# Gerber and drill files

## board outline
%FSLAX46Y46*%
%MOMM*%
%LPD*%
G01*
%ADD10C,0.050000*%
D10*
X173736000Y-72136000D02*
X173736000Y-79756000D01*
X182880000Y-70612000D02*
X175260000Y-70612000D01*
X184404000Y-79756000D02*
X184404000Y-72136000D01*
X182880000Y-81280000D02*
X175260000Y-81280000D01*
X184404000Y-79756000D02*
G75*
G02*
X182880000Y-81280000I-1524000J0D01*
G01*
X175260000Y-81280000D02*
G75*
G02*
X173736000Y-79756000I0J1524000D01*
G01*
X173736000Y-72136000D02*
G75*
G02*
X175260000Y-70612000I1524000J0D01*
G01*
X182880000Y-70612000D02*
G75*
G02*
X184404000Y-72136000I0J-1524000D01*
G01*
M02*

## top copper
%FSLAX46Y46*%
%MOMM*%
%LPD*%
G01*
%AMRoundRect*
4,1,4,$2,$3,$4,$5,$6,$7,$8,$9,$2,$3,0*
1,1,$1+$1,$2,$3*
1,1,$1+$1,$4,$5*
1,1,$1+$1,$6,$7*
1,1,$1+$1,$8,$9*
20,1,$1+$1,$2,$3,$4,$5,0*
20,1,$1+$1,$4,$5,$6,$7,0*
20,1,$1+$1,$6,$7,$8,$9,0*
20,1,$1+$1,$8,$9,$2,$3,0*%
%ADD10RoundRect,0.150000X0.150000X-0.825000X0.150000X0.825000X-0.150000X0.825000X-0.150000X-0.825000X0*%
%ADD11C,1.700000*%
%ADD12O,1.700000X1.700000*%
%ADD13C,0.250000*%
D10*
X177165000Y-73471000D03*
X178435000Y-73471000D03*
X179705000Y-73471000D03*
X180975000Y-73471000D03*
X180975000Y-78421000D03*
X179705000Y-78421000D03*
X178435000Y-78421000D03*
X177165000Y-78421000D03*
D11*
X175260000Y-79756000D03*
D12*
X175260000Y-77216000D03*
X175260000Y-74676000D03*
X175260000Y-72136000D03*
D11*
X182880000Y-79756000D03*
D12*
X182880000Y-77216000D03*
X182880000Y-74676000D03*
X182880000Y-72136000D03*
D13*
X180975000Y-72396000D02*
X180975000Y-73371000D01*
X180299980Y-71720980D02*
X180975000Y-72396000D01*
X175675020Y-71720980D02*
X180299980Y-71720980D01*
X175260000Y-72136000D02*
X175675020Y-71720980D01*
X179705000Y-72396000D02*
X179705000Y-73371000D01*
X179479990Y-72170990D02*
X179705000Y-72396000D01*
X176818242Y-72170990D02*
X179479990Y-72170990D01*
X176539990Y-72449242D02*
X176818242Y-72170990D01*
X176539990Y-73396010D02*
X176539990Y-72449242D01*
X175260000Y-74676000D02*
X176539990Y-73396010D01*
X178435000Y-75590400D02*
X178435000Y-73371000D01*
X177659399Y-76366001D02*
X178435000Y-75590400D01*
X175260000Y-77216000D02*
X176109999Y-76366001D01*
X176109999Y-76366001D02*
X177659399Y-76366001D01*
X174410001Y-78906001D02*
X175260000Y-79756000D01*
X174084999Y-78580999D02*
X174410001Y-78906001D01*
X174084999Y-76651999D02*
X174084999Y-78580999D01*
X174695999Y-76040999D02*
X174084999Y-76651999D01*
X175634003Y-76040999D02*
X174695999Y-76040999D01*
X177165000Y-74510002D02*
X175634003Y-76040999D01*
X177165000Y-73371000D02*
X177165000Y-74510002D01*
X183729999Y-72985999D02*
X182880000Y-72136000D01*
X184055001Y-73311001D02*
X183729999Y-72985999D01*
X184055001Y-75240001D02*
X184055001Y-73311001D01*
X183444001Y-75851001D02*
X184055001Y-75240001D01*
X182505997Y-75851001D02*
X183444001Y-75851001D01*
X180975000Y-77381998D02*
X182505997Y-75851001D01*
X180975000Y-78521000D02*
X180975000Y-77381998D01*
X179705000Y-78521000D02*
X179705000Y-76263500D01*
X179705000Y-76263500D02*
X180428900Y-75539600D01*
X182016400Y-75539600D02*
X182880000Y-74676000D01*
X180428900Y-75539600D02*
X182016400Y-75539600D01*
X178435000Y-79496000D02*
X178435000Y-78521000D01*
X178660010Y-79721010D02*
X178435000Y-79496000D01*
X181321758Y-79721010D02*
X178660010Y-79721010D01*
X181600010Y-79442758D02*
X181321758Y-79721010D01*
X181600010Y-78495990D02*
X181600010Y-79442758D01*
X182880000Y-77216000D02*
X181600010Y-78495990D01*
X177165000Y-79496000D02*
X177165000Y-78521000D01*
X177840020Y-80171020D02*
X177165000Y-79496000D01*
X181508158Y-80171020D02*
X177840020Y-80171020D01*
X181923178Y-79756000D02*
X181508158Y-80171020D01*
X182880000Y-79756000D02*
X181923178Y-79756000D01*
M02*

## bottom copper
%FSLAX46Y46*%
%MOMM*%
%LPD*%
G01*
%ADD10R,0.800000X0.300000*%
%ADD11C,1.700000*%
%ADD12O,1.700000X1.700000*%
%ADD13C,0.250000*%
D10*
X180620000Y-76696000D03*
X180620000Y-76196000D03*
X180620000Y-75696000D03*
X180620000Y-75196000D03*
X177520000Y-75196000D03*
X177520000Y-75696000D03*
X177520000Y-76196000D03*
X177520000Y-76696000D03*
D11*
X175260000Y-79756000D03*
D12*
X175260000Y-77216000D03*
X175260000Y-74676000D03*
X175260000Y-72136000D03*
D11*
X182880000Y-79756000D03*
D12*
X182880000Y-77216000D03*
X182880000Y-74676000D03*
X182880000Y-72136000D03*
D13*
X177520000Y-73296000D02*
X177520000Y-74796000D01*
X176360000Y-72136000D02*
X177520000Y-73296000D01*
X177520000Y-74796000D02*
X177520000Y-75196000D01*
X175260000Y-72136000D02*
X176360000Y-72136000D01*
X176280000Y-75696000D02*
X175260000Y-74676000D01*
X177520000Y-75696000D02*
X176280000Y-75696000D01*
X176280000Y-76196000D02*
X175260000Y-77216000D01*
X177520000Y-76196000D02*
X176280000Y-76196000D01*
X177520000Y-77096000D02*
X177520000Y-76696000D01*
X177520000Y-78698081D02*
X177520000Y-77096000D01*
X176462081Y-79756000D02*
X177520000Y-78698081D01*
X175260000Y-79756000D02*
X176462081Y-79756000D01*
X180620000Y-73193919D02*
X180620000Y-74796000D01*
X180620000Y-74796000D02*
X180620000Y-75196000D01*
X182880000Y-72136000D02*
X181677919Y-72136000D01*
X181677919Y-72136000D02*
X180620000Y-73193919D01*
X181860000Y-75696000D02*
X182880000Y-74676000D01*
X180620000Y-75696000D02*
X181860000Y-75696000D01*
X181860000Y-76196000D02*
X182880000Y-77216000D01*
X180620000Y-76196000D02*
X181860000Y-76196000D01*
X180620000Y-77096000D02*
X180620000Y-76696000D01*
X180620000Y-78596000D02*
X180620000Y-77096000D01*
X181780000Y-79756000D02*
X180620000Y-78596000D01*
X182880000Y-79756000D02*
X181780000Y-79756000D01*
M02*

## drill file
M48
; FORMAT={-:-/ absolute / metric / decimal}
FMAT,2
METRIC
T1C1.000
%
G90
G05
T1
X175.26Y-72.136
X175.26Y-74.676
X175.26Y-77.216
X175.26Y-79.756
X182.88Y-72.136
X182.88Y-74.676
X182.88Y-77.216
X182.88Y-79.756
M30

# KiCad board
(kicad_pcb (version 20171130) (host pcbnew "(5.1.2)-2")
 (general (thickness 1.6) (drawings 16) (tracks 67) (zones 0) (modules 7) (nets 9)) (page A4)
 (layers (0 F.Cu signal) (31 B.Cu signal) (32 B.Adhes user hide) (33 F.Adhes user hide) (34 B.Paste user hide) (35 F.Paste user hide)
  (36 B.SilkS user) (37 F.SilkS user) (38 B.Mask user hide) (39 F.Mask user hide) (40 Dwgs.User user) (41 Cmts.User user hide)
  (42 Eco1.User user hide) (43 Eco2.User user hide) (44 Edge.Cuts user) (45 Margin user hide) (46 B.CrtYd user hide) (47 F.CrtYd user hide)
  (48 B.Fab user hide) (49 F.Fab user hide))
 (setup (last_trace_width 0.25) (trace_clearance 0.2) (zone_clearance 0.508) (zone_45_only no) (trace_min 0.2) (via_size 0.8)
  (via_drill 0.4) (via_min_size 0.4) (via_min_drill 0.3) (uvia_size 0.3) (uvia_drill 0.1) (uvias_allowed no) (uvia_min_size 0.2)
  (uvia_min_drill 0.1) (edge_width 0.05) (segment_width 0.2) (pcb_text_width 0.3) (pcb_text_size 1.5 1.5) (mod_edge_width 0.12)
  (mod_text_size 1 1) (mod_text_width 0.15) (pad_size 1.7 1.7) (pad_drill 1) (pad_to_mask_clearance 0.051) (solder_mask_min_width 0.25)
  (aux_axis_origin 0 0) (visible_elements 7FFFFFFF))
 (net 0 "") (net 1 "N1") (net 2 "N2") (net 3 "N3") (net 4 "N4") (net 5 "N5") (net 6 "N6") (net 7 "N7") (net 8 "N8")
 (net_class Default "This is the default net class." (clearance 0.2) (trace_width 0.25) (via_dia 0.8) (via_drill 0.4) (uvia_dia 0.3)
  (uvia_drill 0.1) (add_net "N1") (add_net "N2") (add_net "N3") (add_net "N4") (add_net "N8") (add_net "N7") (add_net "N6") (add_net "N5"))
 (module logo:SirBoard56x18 (layer B.Cu) (at 179.07 78.867)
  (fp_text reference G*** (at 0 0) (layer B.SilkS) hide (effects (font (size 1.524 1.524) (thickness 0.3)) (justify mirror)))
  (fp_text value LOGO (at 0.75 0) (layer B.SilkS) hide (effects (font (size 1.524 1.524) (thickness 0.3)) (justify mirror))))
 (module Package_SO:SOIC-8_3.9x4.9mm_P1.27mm (layer F.Cu) (at 179.07 75.946 90)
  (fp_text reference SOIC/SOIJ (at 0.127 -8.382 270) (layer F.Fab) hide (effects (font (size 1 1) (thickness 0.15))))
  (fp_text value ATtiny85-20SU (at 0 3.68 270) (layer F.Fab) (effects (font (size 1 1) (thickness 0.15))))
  (pad 8 smd roundrect (at 2.475 -1.905 90) (size 1.95 0.6) (layers F.Cu F.Paste F.Mask) (roundrect_rratio 0.25) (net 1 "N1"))
  (pad 7 smd roundrect (at 2.475 -0.635 90) (size 1.95 0.6) (layers F.Cu F.Paste F.Mask) (roundrect_rratio 0.25) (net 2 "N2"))
  (pad 6 smd roundrect (at 2.475 0.635 90) (size 1.95 0.6) (layers F.Cu F.Paste F.Mask) (roundrect_rratio 0.25) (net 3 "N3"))
  (pad 5 smd roundrect (at 2.475 1.905 90) (size 1.95 0.6) (layers F.Cu F.Paste F.Mask) (roundrect_rratio 0.25) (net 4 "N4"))
  (pad 4 smd roundrect (at -2.475 1.905 90) (size 1.95 0.6) (layers F.Cu F.Paste F.Mask) (roundrect_rratio 0.25) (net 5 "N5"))
  (pad 3 smd roundrect (at -2.475 0.635 90) (size 1.95 0.6) (layers F.Cu F.Paste F.Mask) (roundrect_rratio 0.25) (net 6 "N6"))
  (pad 2 smd roundrect (at -2.475 -0.635 90) (size 1.95 0.6) (layers F.Cu F.Paste F.Mask) (roundrect_rratio 0.25) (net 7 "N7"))
  (pad 1 smd roundrect (at -2.475 -1.905 90) (size 1.95 0.6) (layers F.Cu F.Paste F.Mask) (roundrect_rratio 0.25) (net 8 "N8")))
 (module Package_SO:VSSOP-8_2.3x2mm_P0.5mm (layer B.Cu) (at 179.07 75.946)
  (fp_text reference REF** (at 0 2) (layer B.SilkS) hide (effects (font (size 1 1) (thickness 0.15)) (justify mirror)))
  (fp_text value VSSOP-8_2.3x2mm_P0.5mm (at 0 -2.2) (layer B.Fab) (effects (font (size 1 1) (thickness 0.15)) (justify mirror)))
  (pad 8 smd rect (at 1.55 0.75 90) (size 0.3 0.8) (layers B.Cu B.Paste B.Mask) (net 8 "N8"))
  (pad 7 smd rect (at 1.55 0.25 90) (size 0.3 0.8) (layers B.Cu B.Paste B.Mask) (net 7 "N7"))
  (pad 6 smd rect (at 1.55 -0.25 90) (size 0.3 0.8) (layers B.Cu B.Paste B.Mask) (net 6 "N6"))
  (pad 5 smd rect (at 1.55 -0.75 90) (size 0.3 0.8) (layers B.Cu B.Paste B.Mask) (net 5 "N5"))
  (pad 4 smd rect (at -1.55 -0.75 90) (size 0.3 0.8) (layers B.Cu B.Paste B.Mask) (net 4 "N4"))
  (pad 3 smd rect (at -1.55 -0.25 90) (size 0.3 0.8) (layers B.Cu B.Paste B.Mask) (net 3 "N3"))
  (pad 2 smd rect (at -1.55 0.25 90) (size 0.3 0.8) (layers B.Cu B.Paste B.Mask) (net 2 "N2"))
  (pad 1 smd rect (at -1.55 0.75 90) (size 0.3 0.8) (layers B.Cu B.Paste B.Mask) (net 1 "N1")))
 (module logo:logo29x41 (layer F.Cu) (at 179.07 71.501 90)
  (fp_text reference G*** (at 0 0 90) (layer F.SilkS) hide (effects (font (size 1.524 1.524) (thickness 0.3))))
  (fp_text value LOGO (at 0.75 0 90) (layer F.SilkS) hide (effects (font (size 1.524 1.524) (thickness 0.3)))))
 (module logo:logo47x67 (layer B.Cu) (at 179.07 72.5805 90)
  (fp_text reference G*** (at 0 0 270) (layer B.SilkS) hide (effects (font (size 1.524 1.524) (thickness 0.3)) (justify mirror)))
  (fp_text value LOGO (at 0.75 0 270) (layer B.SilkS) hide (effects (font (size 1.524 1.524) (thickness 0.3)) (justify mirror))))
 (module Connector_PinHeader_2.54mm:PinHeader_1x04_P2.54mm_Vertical (layer B.Cu) (at 175.26 79.756)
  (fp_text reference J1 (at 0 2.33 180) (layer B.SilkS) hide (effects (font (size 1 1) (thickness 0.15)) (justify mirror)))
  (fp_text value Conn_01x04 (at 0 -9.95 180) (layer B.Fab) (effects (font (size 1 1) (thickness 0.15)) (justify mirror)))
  (pad 1 thru_hole circle (at 0 0) (size 1.7 1.7) (drill 1) (layers *.Cu *.Mask) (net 1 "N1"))
  (pad 2 thru_hole oval (at 0 -2.54) (size 1.7 1.7) (drill 1) (layers *.Cu *.Mask) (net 2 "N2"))
  (pad 3 thru_hole oval (at 0 -5.08) (size 1.7 1.7) (drill 1) (layers *.Cu *.Mask) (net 3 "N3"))
  (pad 4 thru_hole oval (at 0 -7.62) (size 1.7 1.7) (drill 1) (layers *.Cu *.Mask) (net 4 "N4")))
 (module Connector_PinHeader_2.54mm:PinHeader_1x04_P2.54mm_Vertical (layer B.Cu) (at 182.88 79.756)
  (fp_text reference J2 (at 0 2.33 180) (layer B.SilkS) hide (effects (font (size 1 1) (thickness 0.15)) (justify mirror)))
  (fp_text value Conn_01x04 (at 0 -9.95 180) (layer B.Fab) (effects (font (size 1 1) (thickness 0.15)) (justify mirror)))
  (pad 1 thru_hole circle (at 0 0) (size 1.7 1.7) (drill 1) (layers *.Cu *.Mask) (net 8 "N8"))
  (pad 2 thru_hole oval (at 0 -2.54) (size 1.7 1.7) (drill 1) (layers *.Cu *.Mask) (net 7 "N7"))
  (pad 3 thru_hole oval (at 0 -5.08) (size 1.7 1.7) (drill 1) (layers *.Cu *.Mask) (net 6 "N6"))
  (pad 4 thru_hole oval (at 0 -7.62) (size 1.7 1.7) (drill 1) (layers *.Cu *.Mask) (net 5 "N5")))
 (gr_line (start 173.736 72.136) (end 173.736 79.756) (layer Edge.Cuts) (width 0.05))
 (gr_line (start 182.88 70.612) (end 175.26 70.612) (layer Edge.Cuts) (width 0.05))
 (gr_line (start 184.404 79.756) (end 184.404 72.136) (layer Edge.Cuts) (width 0.05))
 (gr_line (start 182.88 81.28) (end 175.26 81.28) (layer Edge.Cuts) (width 0.05))
 (gr_arc (start 182.88 79.756) (end 182.88 81.28) (angle -90) (layer Edge.Cuts) (width 0.05))
 (gr_arc (start 175.26 79.756) (end 173.736 79.756) (angle -90) (layer Edge.Cuts) (width 0.05))
 (gr_arc (start 175.26 72.136) (end 175.26 70.612) (angle -90) (layer Edge.Cuts) (width 0.05))
 (gr_arc (start 182.88 72.136) (end 184.404 72.136) (angle -90) (layer Edge.Cuts) (width 0.05))
 (segment (start 180.975 72.396) (end 180.975 73.371) (width 0.25) (layer F.Cu) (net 4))
 (segment (start 180.29998 71.72098) (end 180.975 72.396) (width 0.25) (layer F.Cu) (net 4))
 (segment (start 175.67502 71.72098) (end 180.29998 71.72098) (width 0.25) (layer F.Cu) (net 4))
 (segment (start 175.26 72.136) (end 175.67502 71.72098) (width 0.25) (layer F.Cu) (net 4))
 (segment (start 177.52 73.296) (end 177.52 74.796) (width 0.25) (layer B.Cu) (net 4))
 (segment (start 176.36 72.136) (end 177.52 73.296) (width 0.25) (layer B.Cu) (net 4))
 (segment (start 177.52 74.796) (end 177.52 75.196) (width 0.25) (layer B.Cu) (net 4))
 (segment (start 175.26 72.136) (end 176.36 72.136) (width 0.25) (layer B.Cu) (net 4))
 (segment (start 179.705 72.396) (end 179.705 73.371) (width 0.25) (layer F.Cu) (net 3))
 (segment (start 179.47999 72.17099) (end 179.705 72.396) (width 0.25) (layer F.Cu) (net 3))
 (segment (start 176.818242 72.17099) (end 179.47999 72.17099) (width 0.25) (layer F.Cu) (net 3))
 (segment (start 176.53999 72.449242) (end 176.818242 72.17099) (width 0.25) (layer F.Cu) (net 3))
 (segment (start 176.53999 73.39601) (end 176.53999 72.449242) (width 0.25) (layer F.Cu) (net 3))
 (segment (start 175.26 74.676) (end 176.53999 73.39601) (width 0.25) (layer F.Cu) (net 3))
 (segment (start 176.28 75.696) (end 175.26 74.676) (width 0.25) (layer B.Cu) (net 3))
 (segment (start 177.52 75.696) (end 176.28 75.696) (width 0.25) (layer B.Cu) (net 3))
 (segment (start 178.435 75.5904) (end 178.435 73.371) (width 0.25) (layer F.Cu) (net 2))
 (segment (start 177.659399 76.366001) (end 178.435 75.5904) (width 0.25) (layer F.Cu) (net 2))
 (segment (start 175.26 77.216) (end 176.109999 76.366001) (width 0.25) (layer F.Cu) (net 2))
 (segment (start 176.109999 76.366001) (end 177.659399 76.366001) (width 0.25) (layer F.Cu) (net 2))
 (segment (start 176.28 76.196) (end 175.26 77.216) (width 0.25) (layer B.Cu) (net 2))
 (segment (start 177.52 76.196) (end 176.28 76.196) (width 0.25) (layer B.Cu) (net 2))
 (segment (start 174.410001 78.906001) (end 175.26 79.756) (width 0.25) (layer F.Cu) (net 1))
 (segment (start 174.084999 78.580999) (end 174.410001 78.906001) (width 0.25) (layer F.Cu) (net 1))
 (segment (start 174.084999 76.651999) (end 174.084999 78.580999) (width 0.25) (layer F.Cu) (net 1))
 (segment (start 174.695999 76.040999) (end 174.084999 76.651999) (width 0.25) (layer F.Cu) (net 1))
 (segment (start 175.634003 76.040999) (end 174.695999 76.040999) (width 0.25) (layer F.Cu) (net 1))
 (segment (start 177.165 74.510002) (end 175.634003 76.040999) (width 0.25) (layer F.Cu) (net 1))
 (segment (start 177.165 73.371) (end 177.165 74.510002) (width 0.25) (layer F.Cu) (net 1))
 (segment (start 177.52 77.096) (end 177.52 76.696) (width 0.25) (layer B.Cu) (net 1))
 (segment (start 177.52 78.698081) (end 177.52 77.096) (width 0.25) (layer B.Cu) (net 1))
 (segment (start 176.462081 79.756) (end 177.52 78.698081) (width 0.25) (layer B.Cu) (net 1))
 (segment (start 175.26 79.756) (end 176.462081 79.756) (width 0.25) (layer B.Cu) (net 1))
 (segment (start 180.62 73.193919) (end 180.62 74.796) (width 0.25) (layer B.Cu) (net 5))
 (segment (start 180.62 74.796) (end 180.62 75.196) (width 0.25) (layer B.Cu) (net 5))
 (segment (start 182.88 72.136) (end 181.677919 72.136) (width 0.25) (layer B.Cu) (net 5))
 (segment (start 181.677919 72.136) (end 180.62 73.193919) (width 0.25) (layer B.Cu) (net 5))
 (segment (start 183.729999 72.985999) (end 182.88 72.136) (width 0.25) (layer F.Cu) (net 5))
 (segment (start 184.055001 73.311001) (end 183.729999 72.985999) (width 0.25) (layer F.Cu) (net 5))
 (segment (start 184.055001 75.240001) (end 184.055001 73.311001) (width 0.25) (layer F.Cu) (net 5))
 (segment (start 183.444001 75.851001) (end 184.055001 75.240001) (width 0.25) (layer F.Cu) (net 5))
 (segment (start 182.505997 75.851001) (end 183.444001 75.851001) (width 0.25) (layer F.Cu) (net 5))
 (segment (start 180.975 77.381998) (end 182.505997 75.851001) (width 0.25) (layer F.Cu) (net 5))
 (segment (start 180.975 78.521) (end 180.975 77.381998) (width 0.25) (layer F.Cu) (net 5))
 (segment (start 179.705 78.521) (end 179.705 76.2635) (width 0.25) (layer F.Cu) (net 6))
 (segment (start 179.705 76.2635) (end 180.4289 75.5396) (width 0.25) (layer F.Cu) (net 6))
 (segment (start 182.0164 75.5396) (end 182.88 74.676) (width 0.25) (layer F.Cu) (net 6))
 (segment (start 180.4289 75.5396) (end 182.0164 75.5396) (width 0.25) (layer F.Cu) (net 6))
 (segment (start 181.86 75.696) (end 182.88 74.676) (width 0.25) (layer B.Cu) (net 6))
 (segment (start 180.62 75.696) (end 181.86 75.696) (width 0.25) (layer B.Cu) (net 6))
 (segment (start 178.435 79.496) (end 178.435 78.521) (width 0.25) (layer F.Cu) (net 7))
 (segment (start 178.66001 79.72101) (end 178.435 79.496) (width 0.25) (layer F.Cu) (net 7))
 (segment (start 181.321758 79.72101) (end 178.66001 79.72101) (width 0.25) (layer F.Cu) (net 7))
 (segment (start 181.60001 79.442758) (end 181.321758 79.72101) (width 0.25) (layer F.Cu) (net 7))
 (segment (start 181.60001 78.49599) (end 181.60001 79.442758) (width 0.25) (layer F.Cu) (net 7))
 (segment (start 182.88 77.216) (end 181.60001 78.49599) (width 0.25) (layer F.Cu) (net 7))
 (segment (start 181.86 76.196) (end 182.88 77.216) (width 0.25) (layer B.Cu) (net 7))
 (segment (start 180.62 76.196) (end 181.86 76.196) (width 0.25) (layer B.Cu) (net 7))
 (segment (start 177.165 79.496) (end 177.165 78.521) (width 0.25) (layer F.Cu) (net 8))
 (segment (start 177.84002 80.17102) (end 177.165 79.496) (width 0.25) (layer F.Cu) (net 8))
 (segment (start 181.508158 80.17102) (end 177.84002 80.17102) (width 0.25) (layer F.Cu) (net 8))
 (segment (start 181.923178 79.756) (end 181.508158 80.17102) (width 0.25) (layer F.Cu) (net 8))
 (segment (start 182.88 79.756) (end 181.923178 79.756) (width 0.25) (layer F.Cu) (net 8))
 (segment (start 180.62 77.096) (end 180.62 76.696) (width 0.25) (layer B.Cu) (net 8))
 (segment (start 180.62 78.596) (end 180.62 77.096) (width 0.25) (layer B.Cu) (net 8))
 (segment (start 181.78 79.756) (end 180.62 78.596) (width 0.25) (layer B.Cu) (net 8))
 (segment (start 182.88 79.756) (end 181.78 79.756) (width 0.25) (layer B.Cu) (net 8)))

